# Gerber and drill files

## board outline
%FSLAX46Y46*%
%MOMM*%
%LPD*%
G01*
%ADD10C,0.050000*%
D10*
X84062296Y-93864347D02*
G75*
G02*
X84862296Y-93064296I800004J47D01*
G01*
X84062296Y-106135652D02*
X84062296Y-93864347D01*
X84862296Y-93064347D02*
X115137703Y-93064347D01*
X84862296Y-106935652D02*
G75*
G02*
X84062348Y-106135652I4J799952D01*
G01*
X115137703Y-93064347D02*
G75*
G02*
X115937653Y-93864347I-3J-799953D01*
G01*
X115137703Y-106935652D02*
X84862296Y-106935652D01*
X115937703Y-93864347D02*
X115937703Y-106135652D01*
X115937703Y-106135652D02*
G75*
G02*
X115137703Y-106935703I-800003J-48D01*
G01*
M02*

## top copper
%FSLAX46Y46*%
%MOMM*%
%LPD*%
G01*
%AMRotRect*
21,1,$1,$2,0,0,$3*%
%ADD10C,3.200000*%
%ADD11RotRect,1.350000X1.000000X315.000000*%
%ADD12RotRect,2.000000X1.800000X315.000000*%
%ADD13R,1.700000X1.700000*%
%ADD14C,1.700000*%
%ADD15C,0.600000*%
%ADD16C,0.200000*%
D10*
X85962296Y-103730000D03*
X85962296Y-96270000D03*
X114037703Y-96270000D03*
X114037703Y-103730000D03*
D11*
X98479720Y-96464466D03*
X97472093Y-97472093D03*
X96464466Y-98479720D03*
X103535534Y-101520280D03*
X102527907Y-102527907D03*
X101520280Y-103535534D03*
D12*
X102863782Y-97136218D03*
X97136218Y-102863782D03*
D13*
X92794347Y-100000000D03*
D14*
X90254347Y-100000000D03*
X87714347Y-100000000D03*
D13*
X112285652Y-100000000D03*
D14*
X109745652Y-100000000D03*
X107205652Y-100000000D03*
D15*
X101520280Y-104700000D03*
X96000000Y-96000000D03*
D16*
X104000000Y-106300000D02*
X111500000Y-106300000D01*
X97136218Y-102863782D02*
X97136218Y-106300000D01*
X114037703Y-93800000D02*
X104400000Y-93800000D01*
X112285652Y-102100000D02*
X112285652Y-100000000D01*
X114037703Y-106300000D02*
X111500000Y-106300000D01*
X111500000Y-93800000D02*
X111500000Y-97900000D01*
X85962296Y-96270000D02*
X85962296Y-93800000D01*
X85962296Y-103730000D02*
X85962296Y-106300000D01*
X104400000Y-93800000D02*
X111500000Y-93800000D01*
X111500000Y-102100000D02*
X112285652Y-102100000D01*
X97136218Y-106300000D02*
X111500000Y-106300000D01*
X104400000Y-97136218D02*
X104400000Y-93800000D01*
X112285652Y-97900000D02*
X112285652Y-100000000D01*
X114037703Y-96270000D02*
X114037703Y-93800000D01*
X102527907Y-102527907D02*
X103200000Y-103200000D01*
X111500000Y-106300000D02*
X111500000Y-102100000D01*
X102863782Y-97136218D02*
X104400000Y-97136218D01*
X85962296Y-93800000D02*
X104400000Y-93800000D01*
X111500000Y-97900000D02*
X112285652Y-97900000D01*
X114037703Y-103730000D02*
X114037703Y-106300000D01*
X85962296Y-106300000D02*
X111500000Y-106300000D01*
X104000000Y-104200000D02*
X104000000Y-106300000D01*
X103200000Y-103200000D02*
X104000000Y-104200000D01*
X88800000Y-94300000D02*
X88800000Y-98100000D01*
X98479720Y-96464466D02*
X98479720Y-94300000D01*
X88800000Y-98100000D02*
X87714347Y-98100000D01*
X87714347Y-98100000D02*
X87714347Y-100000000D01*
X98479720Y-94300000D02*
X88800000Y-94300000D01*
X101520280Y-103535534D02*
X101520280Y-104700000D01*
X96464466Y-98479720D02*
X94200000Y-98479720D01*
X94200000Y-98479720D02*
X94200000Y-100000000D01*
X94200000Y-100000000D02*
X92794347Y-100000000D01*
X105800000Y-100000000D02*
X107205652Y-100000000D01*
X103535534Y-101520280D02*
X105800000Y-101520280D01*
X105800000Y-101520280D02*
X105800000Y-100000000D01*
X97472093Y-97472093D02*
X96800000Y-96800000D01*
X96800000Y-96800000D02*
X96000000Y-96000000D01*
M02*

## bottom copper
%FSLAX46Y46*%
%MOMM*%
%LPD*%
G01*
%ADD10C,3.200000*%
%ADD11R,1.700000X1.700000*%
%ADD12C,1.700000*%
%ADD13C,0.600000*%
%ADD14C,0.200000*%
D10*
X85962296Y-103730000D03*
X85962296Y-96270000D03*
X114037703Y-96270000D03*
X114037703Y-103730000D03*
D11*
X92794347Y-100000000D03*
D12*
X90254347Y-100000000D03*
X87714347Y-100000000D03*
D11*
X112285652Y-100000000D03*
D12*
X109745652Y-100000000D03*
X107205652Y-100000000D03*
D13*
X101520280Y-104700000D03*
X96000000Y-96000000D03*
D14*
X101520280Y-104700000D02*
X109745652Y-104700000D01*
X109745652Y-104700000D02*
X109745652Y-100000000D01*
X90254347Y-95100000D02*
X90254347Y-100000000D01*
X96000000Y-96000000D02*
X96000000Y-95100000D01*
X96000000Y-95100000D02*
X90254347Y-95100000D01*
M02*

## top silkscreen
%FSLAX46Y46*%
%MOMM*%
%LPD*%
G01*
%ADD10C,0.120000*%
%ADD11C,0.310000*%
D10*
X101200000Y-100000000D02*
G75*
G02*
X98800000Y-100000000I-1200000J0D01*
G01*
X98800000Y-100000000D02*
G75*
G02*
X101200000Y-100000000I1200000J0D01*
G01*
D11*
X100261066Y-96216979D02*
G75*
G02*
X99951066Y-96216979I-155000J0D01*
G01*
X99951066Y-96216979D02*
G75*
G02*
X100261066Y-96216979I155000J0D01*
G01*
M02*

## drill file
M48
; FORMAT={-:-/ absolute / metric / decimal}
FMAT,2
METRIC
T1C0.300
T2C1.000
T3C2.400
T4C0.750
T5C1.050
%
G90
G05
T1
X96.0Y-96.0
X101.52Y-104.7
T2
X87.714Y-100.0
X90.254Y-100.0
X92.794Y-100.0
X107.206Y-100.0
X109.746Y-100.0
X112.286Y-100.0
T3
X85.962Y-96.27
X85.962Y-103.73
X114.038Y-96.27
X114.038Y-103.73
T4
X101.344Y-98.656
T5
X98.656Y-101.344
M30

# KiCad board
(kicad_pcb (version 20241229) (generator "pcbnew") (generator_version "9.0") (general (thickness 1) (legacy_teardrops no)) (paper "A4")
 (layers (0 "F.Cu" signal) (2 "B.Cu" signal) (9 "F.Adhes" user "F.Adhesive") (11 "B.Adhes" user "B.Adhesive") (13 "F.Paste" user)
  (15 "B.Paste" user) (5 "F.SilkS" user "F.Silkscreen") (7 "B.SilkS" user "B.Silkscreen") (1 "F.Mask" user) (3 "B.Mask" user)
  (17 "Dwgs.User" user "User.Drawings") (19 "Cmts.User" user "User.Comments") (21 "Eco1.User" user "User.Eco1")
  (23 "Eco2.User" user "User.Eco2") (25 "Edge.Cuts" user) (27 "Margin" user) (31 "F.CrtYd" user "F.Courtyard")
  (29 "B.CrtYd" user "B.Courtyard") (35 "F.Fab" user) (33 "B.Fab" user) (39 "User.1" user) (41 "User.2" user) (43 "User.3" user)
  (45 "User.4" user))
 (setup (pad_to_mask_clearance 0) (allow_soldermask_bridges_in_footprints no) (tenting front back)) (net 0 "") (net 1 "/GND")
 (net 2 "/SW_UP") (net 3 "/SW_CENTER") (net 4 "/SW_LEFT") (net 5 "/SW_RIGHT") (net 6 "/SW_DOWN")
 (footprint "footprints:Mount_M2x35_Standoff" (layer "F.Cu") (at 85.962296 103.73)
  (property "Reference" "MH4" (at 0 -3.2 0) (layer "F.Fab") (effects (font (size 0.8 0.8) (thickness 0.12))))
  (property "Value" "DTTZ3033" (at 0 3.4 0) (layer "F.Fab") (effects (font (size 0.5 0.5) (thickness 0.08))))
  (pad "1" thru_hole circle (at 0 0) (size 3.2 3.2) (drill 2.4) (layers "*.Cu" "*.Mask") (remove_unused_layers no) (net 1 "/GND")))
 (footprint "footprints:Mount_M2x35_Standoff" (layer "F.Cu") (at 85.962296 96.27)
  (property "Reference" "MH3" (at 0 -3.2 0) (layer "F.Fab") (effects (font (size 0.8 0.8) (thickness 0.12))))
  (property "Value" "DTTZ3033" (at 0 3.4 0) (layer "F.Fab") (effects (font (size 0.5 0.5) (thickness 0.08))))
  (pad "1" thru_hole circle (at 0 0) (size 3.2 3.2) (drill 2.4) (layers "*.Cu" "*.Mask") (remove_unused_layers no) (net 1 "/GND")))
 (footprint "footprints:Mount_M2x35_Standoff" (layer "F.Cu") (at 114.037703 96.27)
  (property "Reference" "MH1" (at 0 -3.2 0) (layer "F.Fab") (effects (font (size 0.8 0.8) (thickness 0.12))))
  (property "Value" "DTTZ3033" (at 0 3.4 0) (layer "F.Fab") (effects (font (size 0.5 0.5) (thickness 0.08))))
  (pad "1" thru_hole circle (at 0 0) (size 3.2 3.2) (drill 2.4) (layers "*.Cu" "*.Mask") (remove_unused_layers no) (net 1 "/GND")))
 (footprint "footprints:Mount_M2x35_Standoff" (layer "F.Cu") (at 114.037703 103.73)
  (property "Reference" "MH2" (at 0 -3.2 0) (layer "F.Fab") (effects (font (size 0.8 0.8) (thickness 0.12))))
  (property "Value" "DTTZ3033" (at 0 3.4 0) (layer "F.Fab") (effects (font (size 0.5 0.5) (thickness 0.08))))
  (pad "1" thru_hole circle (at 0 0) (size 3.2 3.2) (drill 2.4) (layers "*.Cu" "*.Mask") (remove_unused_layers no) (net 1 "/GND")))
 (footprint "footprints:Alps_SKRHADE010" (layer "F.Cu") (at 100 100 -45)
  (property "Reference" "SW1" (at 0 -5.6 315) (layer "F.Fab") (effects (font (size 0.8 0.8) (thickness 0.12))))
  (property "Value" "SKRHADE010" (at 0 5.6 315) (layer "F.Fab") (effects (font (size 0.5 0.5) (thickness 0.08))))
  (fp_circle (center 0 0) (end 1.2 0) (stroke (width 0.12) (type solid)) (fill no) (layer "F.SilkS"))
  (fp_circle (center -2.6 -2.75) (end -2.35 -2.75) (stroke (width 0.12) (type solid)) (fill yes) (layer "F.SilkS"))
  (pad "" np_thru_hole circle (at 0 -1.9 315) (size 0.75 0.75) (drill 0.75) (layers "*.Cu" "*.Mask"))
  (pad "" np_thru_hole circle (at 0 1.9 315) (size 1.05 1.05) (drill 1.05) (layers "*.Cu" "*.Mask"))
  (pad "1" smd rect (at -3.575 -1.425 315) (size 1.35 1) (layers "F.Cu" "F.Mask" "F.Paste") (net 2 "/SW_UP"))
  (pad "2" smd rect (at -3.575 0 315) (size 1.35 1) (layers "F.Cu" "F.Mask" "F.Paste") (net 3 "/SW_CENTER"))
  (pad "3" smd rect (at -3.575 1.425 315) (size 1.35 1) (layers "F.Cu" "F.Mask" "F.Paste") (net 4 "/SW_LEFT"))
  (pad "4" smd rect (at 3.575 -1.425 315) (size 1.35 1) (layers "F.Cu" "F.Mask" "F.Paste") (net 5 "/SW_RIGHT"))
  (pad "5" smd rect (at 3.575 0 315) (size 1.35 1) (layers "F.Cu" "F.Mask" "F.Paste") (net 1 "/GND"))
  (pad "6" smd rect (at 3.575 1.425 315) (size 1.35 1) (layers "F.Cu" "F.Mask" "F.Paste") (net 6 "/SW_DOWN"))
  (pad "7" smd rect (at 0 -4.049999 315) (size 2 1.8) (layers "F.Cu" "F.Mask" "F.Paste") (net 1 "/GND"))
  (pad "8" smd rect (at 0 4.049999 315) (size 2 1.8) (layers "F.Cu" "F.Mask" "F.Paste") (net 1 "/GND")))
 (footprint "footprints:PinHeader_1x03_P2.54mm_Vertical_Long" (layer "B.Cu") (at 90.254347 100 180)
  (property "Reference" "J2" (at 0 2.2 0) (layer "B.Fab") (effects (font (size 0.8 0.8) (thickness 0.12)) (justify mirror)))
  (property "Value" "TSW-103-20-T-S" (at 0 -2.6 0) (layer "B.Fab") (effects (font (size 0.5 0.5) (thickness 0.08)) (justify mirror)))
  (pad "1" thru_hole rect (at -2.54 0 180) (size 1.7 1.7) (drill 1) (layers "*.Cu" "*.Mask") (remove_unused_layers no) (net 4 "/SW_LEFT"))
  (pad "2" thru_hole circle (at 0 0 180) (size 1.7 1.7) (drill 1) (layers "*.Cu" "*.Mask") (remove_unused_layers no) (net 3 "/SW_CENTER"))
  (pad "3" thru_hole circle (at 2.54 0 180) (size 1.7 1.7) (drill 1) (layers "*.Cu" "*.Mask") (remove_unused_layers no) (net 2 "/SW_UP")))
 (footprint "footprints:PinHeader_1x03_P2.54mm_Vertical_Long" (layer "B.Cu") (at 109.745652 100 180)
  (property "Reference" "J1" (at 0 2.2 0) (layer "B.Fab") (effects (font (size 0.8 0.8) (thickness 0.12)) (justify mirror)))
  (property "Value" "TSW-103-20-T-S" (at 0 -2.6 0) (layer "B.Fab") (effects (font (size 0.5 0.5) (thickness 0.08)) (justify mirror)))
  (pad "1" thru_hole rect (at -2.54 0 180) (size 1.7 1.7) (drill 1) (layers "*.Cu" "*.Mask") (remove_unused_layers no) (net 1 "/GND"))
  (pad "2" thru_hole circle (at 0 0 180) (size 1.7 1.7) (drill 1) (layers "*.Cu" "*.Mask") (remove_unused_layers no) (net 6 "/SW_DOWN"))
  (pad "3" thru_hole circle (at 2.54 0 180) (size 1.7 1.7) (drill 1) (layers "*.Cu" "*.Mask") (remove_unused_layers no) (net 5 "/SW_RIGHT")))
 (gr_arc (start 84.062296 93.864347) (mid 84.296611 93.298662) (end 84.862296 93.064347) (stroke (width 0.05) (type default))
  (layer "Edge.Cuts"))
 (gr_line (start 84.062296 106.135652) (end 84.062296 93.864347) (stroke (width 0.05) (type default)) (layer "Edge.Cuts"))
 (gr_line (start 84.862296 93.064347) (end 115.137703 93.064347) (stroke (width 0.05) (type default)) (layer "Edge.Cuts"))
 (gr_arc (start 84.862296 106.935652) (mid 84.296611 106.701337) (end 84.062296 106.135652) (stroke (width 0.05) (type default))
  (layer "Edge.Cuts"))
 (gr_arc (start 115.137703 93.064347) (mid 115.703388 93.298662) (end 115.937703 93.864347) (stroke (width 0.05) (type default))
  (layer "Edge.Cuts"))
 (gr_line (start 115.137703 106.935652) (end 84.862296 106.935652) (stroke (width 0.05) (type default)) (layer "Edge.Cuts"))
 (gr_line (start 115.937703 93.864347) (end 115.937703 106.135652) (stroke (width 0.05) (type default)) (layer "Edge.Cuts"))
 (gr_arc (start 115.937703 106.135652) (mid 115.703388 106.701337) (end 115.137703 106.935652) (stroke (width 0.05) (type default))
  (layer "Edge.Cuts"))
 (segment (start 104 106.3) (end 111.5 106.3) (width 0.2) (layer "F.Cu") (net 1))
 (segment (start 97.136218 102.863782) (end 97.136218 106.3) (width 0.2) (layer "F.Cu") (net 1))
 (segment (start 114.037703 93.8) (end 104.4 93.8) (width 0.2) (layer "F.Cu") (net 1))
 (segment (start 112.285652 102.1) (end 112.285652 100) (width 0.2) (layer "F.Cu") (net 1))
 (segment (start 114.037703 106.3) (end 111.5 106.3) (width 0.2) (layer "F.Cu") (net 1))
 (segment (start 111.5 93.8) (end 111.5 97.9) (width 0.2) (layer "F.Cu") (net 1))
 (segment (start 85.962296 96.27) (end 85.962296 93.8) (width 0.2) (layer "F.Cu") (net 1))
 (segment (start 85.962296 103.73) (end 85.962296 106.3) (width 0.2) (layer "F.Cu") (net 1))
 (segment (start 104.4 93.8) (end 111.5 93.8) (width 0.2) (layer "F.Cu") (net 1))
 (segment (start 111.5 102.1) (end 112.285652 102.1) (width 0.2) (layer "F.Cu") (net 1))
 (segment (start 97.136218 106.3) (end 111.5 106.3) (width 0.2) (layer "F.Cu") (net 1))
 (segment (start 104.4 97.136218) (end 104.4 93.8) (width 0.2) (layer "F.Cu") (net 1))
 (segment (start 112.285652 97.9) (end 112.285652 100) (width 0.2) (layer "F.Cu") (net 1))
 (segment (start 114.037703 96.27) (end 114.037703 93.8) (width 0.2) (layer "F.Cu") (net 1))
 (segment (start 102.527907 102.527907) (end 103.2 103.2) (width 0.2) (layer "F.Cu") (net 1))
 (segment (start 111.5 106.3) (end 111.5 102.1) (width 0.2) (layer "F.Cu") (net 1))
 (segment (start 102.863782 97.136218) (end 104.4 97.136218) (width 0.2) (layer "F.Cu") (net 1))
 (segment (start 85.962296 93.8) (end 104.4 93.8) (width 0.2) (layer "F.Cu") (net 1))
 (segment (start 111.5 97.9) (end 112.285652 97.9) (width 0.2) (layer "F.Cu") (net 1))
 (segment (start 114.037703 103.73) (end 114.037703 106.3) (width 0.2) (layer "F.Cu") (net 1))
 (segment (start 85.962296 106.3) (end 111.5 106.3) (width 0.2) (layer "F.Cu") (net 1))
 (segment (start 104 104.2) (end 104 106.3) (width 0.2) (layer "F.Cu") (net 1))
 (segment (start 103.2 103.2) (end 104 104.2) (width 0.2) (layer "F.Cu") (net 1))
 (segment (start 88.8 94.3) (end 88.8 98.1) (width 0.2) (layer "F.Cu") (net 2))
 (segment (start 98.47972 96.464466) (end 98.47972 94.3) (width 0.2) (layer "F.Cu") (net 2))
 (segment (start 88.8 98.1) (end 87.714347 98.1) (width 0.2) (layer "F.Cu") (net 2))
 (segment (start 87.714347 98.1) (end 87.714347 100) (width 0.2) (layer "F.Cu") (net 2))
 (segment (start 98.47972 94.3) (end 88.8 94.3) (width 0.2) (layer "F.Cu") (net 2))
 (segment (start 101.52028 103.535534) (end 101.52028 104.7) (width 0.2) (layer "F.Cu") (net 6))
 (via (at 101.52028 104.7) (size 0.6) (drill 0.3) (layers "F.Cu" "B.Cu") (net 6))
 (segment (start 101.52028 104.7) (end 109.745652 104.7) (width 0.2) (layer "B.Cu") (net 6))
 (segment (start 109.745652 104.7) (end 109.745652 100) (width 0.2) (layer "B.Cu") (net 6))
 (segment (start 96.464466 98.47972) (end 94.2 98.47972) (width 0.2) (layer "F.Cu") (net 4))
 (segment (start 94.2 98.47972) (end 94.2 100) (width 0.2) (layer "F.Cu") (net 4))
 (segment (start 94.2 100) (end 92.794347 100) (width 0.2) (layer "F.Cu") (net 4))
 (segment (start 105.8 100) (end 107.205652 100) (width 0.2) (layer "F.Cu") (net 5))
 (segment (start 103.535534 101.52028) (end 105.8 101.52028) (width 0.2) (layer "F.Cu") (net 5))
 (segment (start 105.8 101.52028) (end 105.8 100) (width 0.2) (layer "F.Cu") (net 5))
 (segment (start 97.472093 97.472093) (end 96.8 96.8) (width 0.2) (layer "F.Cu") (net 3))
 (segment (start 96.8 96.8) (end 96 96) (width 0.2) (layer "F.Cu") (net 3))
 (via (at 96 96) (size 0.6) (drill 0.3) (layers "F.Cu" "B.Cu") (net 3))
 (segment (start 90.254347 95.1) (end 90.254347 100) (width 0.2) (layer "B.Cu") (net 3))
 (segment (start 96 96) (end 96 95.1) (width 0.2) (layer "B.Cu") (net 3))
 (segment (start 96 95.1) (end 90.254347 95.1) (width 0.2) (layer "B.Cu") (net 3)))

